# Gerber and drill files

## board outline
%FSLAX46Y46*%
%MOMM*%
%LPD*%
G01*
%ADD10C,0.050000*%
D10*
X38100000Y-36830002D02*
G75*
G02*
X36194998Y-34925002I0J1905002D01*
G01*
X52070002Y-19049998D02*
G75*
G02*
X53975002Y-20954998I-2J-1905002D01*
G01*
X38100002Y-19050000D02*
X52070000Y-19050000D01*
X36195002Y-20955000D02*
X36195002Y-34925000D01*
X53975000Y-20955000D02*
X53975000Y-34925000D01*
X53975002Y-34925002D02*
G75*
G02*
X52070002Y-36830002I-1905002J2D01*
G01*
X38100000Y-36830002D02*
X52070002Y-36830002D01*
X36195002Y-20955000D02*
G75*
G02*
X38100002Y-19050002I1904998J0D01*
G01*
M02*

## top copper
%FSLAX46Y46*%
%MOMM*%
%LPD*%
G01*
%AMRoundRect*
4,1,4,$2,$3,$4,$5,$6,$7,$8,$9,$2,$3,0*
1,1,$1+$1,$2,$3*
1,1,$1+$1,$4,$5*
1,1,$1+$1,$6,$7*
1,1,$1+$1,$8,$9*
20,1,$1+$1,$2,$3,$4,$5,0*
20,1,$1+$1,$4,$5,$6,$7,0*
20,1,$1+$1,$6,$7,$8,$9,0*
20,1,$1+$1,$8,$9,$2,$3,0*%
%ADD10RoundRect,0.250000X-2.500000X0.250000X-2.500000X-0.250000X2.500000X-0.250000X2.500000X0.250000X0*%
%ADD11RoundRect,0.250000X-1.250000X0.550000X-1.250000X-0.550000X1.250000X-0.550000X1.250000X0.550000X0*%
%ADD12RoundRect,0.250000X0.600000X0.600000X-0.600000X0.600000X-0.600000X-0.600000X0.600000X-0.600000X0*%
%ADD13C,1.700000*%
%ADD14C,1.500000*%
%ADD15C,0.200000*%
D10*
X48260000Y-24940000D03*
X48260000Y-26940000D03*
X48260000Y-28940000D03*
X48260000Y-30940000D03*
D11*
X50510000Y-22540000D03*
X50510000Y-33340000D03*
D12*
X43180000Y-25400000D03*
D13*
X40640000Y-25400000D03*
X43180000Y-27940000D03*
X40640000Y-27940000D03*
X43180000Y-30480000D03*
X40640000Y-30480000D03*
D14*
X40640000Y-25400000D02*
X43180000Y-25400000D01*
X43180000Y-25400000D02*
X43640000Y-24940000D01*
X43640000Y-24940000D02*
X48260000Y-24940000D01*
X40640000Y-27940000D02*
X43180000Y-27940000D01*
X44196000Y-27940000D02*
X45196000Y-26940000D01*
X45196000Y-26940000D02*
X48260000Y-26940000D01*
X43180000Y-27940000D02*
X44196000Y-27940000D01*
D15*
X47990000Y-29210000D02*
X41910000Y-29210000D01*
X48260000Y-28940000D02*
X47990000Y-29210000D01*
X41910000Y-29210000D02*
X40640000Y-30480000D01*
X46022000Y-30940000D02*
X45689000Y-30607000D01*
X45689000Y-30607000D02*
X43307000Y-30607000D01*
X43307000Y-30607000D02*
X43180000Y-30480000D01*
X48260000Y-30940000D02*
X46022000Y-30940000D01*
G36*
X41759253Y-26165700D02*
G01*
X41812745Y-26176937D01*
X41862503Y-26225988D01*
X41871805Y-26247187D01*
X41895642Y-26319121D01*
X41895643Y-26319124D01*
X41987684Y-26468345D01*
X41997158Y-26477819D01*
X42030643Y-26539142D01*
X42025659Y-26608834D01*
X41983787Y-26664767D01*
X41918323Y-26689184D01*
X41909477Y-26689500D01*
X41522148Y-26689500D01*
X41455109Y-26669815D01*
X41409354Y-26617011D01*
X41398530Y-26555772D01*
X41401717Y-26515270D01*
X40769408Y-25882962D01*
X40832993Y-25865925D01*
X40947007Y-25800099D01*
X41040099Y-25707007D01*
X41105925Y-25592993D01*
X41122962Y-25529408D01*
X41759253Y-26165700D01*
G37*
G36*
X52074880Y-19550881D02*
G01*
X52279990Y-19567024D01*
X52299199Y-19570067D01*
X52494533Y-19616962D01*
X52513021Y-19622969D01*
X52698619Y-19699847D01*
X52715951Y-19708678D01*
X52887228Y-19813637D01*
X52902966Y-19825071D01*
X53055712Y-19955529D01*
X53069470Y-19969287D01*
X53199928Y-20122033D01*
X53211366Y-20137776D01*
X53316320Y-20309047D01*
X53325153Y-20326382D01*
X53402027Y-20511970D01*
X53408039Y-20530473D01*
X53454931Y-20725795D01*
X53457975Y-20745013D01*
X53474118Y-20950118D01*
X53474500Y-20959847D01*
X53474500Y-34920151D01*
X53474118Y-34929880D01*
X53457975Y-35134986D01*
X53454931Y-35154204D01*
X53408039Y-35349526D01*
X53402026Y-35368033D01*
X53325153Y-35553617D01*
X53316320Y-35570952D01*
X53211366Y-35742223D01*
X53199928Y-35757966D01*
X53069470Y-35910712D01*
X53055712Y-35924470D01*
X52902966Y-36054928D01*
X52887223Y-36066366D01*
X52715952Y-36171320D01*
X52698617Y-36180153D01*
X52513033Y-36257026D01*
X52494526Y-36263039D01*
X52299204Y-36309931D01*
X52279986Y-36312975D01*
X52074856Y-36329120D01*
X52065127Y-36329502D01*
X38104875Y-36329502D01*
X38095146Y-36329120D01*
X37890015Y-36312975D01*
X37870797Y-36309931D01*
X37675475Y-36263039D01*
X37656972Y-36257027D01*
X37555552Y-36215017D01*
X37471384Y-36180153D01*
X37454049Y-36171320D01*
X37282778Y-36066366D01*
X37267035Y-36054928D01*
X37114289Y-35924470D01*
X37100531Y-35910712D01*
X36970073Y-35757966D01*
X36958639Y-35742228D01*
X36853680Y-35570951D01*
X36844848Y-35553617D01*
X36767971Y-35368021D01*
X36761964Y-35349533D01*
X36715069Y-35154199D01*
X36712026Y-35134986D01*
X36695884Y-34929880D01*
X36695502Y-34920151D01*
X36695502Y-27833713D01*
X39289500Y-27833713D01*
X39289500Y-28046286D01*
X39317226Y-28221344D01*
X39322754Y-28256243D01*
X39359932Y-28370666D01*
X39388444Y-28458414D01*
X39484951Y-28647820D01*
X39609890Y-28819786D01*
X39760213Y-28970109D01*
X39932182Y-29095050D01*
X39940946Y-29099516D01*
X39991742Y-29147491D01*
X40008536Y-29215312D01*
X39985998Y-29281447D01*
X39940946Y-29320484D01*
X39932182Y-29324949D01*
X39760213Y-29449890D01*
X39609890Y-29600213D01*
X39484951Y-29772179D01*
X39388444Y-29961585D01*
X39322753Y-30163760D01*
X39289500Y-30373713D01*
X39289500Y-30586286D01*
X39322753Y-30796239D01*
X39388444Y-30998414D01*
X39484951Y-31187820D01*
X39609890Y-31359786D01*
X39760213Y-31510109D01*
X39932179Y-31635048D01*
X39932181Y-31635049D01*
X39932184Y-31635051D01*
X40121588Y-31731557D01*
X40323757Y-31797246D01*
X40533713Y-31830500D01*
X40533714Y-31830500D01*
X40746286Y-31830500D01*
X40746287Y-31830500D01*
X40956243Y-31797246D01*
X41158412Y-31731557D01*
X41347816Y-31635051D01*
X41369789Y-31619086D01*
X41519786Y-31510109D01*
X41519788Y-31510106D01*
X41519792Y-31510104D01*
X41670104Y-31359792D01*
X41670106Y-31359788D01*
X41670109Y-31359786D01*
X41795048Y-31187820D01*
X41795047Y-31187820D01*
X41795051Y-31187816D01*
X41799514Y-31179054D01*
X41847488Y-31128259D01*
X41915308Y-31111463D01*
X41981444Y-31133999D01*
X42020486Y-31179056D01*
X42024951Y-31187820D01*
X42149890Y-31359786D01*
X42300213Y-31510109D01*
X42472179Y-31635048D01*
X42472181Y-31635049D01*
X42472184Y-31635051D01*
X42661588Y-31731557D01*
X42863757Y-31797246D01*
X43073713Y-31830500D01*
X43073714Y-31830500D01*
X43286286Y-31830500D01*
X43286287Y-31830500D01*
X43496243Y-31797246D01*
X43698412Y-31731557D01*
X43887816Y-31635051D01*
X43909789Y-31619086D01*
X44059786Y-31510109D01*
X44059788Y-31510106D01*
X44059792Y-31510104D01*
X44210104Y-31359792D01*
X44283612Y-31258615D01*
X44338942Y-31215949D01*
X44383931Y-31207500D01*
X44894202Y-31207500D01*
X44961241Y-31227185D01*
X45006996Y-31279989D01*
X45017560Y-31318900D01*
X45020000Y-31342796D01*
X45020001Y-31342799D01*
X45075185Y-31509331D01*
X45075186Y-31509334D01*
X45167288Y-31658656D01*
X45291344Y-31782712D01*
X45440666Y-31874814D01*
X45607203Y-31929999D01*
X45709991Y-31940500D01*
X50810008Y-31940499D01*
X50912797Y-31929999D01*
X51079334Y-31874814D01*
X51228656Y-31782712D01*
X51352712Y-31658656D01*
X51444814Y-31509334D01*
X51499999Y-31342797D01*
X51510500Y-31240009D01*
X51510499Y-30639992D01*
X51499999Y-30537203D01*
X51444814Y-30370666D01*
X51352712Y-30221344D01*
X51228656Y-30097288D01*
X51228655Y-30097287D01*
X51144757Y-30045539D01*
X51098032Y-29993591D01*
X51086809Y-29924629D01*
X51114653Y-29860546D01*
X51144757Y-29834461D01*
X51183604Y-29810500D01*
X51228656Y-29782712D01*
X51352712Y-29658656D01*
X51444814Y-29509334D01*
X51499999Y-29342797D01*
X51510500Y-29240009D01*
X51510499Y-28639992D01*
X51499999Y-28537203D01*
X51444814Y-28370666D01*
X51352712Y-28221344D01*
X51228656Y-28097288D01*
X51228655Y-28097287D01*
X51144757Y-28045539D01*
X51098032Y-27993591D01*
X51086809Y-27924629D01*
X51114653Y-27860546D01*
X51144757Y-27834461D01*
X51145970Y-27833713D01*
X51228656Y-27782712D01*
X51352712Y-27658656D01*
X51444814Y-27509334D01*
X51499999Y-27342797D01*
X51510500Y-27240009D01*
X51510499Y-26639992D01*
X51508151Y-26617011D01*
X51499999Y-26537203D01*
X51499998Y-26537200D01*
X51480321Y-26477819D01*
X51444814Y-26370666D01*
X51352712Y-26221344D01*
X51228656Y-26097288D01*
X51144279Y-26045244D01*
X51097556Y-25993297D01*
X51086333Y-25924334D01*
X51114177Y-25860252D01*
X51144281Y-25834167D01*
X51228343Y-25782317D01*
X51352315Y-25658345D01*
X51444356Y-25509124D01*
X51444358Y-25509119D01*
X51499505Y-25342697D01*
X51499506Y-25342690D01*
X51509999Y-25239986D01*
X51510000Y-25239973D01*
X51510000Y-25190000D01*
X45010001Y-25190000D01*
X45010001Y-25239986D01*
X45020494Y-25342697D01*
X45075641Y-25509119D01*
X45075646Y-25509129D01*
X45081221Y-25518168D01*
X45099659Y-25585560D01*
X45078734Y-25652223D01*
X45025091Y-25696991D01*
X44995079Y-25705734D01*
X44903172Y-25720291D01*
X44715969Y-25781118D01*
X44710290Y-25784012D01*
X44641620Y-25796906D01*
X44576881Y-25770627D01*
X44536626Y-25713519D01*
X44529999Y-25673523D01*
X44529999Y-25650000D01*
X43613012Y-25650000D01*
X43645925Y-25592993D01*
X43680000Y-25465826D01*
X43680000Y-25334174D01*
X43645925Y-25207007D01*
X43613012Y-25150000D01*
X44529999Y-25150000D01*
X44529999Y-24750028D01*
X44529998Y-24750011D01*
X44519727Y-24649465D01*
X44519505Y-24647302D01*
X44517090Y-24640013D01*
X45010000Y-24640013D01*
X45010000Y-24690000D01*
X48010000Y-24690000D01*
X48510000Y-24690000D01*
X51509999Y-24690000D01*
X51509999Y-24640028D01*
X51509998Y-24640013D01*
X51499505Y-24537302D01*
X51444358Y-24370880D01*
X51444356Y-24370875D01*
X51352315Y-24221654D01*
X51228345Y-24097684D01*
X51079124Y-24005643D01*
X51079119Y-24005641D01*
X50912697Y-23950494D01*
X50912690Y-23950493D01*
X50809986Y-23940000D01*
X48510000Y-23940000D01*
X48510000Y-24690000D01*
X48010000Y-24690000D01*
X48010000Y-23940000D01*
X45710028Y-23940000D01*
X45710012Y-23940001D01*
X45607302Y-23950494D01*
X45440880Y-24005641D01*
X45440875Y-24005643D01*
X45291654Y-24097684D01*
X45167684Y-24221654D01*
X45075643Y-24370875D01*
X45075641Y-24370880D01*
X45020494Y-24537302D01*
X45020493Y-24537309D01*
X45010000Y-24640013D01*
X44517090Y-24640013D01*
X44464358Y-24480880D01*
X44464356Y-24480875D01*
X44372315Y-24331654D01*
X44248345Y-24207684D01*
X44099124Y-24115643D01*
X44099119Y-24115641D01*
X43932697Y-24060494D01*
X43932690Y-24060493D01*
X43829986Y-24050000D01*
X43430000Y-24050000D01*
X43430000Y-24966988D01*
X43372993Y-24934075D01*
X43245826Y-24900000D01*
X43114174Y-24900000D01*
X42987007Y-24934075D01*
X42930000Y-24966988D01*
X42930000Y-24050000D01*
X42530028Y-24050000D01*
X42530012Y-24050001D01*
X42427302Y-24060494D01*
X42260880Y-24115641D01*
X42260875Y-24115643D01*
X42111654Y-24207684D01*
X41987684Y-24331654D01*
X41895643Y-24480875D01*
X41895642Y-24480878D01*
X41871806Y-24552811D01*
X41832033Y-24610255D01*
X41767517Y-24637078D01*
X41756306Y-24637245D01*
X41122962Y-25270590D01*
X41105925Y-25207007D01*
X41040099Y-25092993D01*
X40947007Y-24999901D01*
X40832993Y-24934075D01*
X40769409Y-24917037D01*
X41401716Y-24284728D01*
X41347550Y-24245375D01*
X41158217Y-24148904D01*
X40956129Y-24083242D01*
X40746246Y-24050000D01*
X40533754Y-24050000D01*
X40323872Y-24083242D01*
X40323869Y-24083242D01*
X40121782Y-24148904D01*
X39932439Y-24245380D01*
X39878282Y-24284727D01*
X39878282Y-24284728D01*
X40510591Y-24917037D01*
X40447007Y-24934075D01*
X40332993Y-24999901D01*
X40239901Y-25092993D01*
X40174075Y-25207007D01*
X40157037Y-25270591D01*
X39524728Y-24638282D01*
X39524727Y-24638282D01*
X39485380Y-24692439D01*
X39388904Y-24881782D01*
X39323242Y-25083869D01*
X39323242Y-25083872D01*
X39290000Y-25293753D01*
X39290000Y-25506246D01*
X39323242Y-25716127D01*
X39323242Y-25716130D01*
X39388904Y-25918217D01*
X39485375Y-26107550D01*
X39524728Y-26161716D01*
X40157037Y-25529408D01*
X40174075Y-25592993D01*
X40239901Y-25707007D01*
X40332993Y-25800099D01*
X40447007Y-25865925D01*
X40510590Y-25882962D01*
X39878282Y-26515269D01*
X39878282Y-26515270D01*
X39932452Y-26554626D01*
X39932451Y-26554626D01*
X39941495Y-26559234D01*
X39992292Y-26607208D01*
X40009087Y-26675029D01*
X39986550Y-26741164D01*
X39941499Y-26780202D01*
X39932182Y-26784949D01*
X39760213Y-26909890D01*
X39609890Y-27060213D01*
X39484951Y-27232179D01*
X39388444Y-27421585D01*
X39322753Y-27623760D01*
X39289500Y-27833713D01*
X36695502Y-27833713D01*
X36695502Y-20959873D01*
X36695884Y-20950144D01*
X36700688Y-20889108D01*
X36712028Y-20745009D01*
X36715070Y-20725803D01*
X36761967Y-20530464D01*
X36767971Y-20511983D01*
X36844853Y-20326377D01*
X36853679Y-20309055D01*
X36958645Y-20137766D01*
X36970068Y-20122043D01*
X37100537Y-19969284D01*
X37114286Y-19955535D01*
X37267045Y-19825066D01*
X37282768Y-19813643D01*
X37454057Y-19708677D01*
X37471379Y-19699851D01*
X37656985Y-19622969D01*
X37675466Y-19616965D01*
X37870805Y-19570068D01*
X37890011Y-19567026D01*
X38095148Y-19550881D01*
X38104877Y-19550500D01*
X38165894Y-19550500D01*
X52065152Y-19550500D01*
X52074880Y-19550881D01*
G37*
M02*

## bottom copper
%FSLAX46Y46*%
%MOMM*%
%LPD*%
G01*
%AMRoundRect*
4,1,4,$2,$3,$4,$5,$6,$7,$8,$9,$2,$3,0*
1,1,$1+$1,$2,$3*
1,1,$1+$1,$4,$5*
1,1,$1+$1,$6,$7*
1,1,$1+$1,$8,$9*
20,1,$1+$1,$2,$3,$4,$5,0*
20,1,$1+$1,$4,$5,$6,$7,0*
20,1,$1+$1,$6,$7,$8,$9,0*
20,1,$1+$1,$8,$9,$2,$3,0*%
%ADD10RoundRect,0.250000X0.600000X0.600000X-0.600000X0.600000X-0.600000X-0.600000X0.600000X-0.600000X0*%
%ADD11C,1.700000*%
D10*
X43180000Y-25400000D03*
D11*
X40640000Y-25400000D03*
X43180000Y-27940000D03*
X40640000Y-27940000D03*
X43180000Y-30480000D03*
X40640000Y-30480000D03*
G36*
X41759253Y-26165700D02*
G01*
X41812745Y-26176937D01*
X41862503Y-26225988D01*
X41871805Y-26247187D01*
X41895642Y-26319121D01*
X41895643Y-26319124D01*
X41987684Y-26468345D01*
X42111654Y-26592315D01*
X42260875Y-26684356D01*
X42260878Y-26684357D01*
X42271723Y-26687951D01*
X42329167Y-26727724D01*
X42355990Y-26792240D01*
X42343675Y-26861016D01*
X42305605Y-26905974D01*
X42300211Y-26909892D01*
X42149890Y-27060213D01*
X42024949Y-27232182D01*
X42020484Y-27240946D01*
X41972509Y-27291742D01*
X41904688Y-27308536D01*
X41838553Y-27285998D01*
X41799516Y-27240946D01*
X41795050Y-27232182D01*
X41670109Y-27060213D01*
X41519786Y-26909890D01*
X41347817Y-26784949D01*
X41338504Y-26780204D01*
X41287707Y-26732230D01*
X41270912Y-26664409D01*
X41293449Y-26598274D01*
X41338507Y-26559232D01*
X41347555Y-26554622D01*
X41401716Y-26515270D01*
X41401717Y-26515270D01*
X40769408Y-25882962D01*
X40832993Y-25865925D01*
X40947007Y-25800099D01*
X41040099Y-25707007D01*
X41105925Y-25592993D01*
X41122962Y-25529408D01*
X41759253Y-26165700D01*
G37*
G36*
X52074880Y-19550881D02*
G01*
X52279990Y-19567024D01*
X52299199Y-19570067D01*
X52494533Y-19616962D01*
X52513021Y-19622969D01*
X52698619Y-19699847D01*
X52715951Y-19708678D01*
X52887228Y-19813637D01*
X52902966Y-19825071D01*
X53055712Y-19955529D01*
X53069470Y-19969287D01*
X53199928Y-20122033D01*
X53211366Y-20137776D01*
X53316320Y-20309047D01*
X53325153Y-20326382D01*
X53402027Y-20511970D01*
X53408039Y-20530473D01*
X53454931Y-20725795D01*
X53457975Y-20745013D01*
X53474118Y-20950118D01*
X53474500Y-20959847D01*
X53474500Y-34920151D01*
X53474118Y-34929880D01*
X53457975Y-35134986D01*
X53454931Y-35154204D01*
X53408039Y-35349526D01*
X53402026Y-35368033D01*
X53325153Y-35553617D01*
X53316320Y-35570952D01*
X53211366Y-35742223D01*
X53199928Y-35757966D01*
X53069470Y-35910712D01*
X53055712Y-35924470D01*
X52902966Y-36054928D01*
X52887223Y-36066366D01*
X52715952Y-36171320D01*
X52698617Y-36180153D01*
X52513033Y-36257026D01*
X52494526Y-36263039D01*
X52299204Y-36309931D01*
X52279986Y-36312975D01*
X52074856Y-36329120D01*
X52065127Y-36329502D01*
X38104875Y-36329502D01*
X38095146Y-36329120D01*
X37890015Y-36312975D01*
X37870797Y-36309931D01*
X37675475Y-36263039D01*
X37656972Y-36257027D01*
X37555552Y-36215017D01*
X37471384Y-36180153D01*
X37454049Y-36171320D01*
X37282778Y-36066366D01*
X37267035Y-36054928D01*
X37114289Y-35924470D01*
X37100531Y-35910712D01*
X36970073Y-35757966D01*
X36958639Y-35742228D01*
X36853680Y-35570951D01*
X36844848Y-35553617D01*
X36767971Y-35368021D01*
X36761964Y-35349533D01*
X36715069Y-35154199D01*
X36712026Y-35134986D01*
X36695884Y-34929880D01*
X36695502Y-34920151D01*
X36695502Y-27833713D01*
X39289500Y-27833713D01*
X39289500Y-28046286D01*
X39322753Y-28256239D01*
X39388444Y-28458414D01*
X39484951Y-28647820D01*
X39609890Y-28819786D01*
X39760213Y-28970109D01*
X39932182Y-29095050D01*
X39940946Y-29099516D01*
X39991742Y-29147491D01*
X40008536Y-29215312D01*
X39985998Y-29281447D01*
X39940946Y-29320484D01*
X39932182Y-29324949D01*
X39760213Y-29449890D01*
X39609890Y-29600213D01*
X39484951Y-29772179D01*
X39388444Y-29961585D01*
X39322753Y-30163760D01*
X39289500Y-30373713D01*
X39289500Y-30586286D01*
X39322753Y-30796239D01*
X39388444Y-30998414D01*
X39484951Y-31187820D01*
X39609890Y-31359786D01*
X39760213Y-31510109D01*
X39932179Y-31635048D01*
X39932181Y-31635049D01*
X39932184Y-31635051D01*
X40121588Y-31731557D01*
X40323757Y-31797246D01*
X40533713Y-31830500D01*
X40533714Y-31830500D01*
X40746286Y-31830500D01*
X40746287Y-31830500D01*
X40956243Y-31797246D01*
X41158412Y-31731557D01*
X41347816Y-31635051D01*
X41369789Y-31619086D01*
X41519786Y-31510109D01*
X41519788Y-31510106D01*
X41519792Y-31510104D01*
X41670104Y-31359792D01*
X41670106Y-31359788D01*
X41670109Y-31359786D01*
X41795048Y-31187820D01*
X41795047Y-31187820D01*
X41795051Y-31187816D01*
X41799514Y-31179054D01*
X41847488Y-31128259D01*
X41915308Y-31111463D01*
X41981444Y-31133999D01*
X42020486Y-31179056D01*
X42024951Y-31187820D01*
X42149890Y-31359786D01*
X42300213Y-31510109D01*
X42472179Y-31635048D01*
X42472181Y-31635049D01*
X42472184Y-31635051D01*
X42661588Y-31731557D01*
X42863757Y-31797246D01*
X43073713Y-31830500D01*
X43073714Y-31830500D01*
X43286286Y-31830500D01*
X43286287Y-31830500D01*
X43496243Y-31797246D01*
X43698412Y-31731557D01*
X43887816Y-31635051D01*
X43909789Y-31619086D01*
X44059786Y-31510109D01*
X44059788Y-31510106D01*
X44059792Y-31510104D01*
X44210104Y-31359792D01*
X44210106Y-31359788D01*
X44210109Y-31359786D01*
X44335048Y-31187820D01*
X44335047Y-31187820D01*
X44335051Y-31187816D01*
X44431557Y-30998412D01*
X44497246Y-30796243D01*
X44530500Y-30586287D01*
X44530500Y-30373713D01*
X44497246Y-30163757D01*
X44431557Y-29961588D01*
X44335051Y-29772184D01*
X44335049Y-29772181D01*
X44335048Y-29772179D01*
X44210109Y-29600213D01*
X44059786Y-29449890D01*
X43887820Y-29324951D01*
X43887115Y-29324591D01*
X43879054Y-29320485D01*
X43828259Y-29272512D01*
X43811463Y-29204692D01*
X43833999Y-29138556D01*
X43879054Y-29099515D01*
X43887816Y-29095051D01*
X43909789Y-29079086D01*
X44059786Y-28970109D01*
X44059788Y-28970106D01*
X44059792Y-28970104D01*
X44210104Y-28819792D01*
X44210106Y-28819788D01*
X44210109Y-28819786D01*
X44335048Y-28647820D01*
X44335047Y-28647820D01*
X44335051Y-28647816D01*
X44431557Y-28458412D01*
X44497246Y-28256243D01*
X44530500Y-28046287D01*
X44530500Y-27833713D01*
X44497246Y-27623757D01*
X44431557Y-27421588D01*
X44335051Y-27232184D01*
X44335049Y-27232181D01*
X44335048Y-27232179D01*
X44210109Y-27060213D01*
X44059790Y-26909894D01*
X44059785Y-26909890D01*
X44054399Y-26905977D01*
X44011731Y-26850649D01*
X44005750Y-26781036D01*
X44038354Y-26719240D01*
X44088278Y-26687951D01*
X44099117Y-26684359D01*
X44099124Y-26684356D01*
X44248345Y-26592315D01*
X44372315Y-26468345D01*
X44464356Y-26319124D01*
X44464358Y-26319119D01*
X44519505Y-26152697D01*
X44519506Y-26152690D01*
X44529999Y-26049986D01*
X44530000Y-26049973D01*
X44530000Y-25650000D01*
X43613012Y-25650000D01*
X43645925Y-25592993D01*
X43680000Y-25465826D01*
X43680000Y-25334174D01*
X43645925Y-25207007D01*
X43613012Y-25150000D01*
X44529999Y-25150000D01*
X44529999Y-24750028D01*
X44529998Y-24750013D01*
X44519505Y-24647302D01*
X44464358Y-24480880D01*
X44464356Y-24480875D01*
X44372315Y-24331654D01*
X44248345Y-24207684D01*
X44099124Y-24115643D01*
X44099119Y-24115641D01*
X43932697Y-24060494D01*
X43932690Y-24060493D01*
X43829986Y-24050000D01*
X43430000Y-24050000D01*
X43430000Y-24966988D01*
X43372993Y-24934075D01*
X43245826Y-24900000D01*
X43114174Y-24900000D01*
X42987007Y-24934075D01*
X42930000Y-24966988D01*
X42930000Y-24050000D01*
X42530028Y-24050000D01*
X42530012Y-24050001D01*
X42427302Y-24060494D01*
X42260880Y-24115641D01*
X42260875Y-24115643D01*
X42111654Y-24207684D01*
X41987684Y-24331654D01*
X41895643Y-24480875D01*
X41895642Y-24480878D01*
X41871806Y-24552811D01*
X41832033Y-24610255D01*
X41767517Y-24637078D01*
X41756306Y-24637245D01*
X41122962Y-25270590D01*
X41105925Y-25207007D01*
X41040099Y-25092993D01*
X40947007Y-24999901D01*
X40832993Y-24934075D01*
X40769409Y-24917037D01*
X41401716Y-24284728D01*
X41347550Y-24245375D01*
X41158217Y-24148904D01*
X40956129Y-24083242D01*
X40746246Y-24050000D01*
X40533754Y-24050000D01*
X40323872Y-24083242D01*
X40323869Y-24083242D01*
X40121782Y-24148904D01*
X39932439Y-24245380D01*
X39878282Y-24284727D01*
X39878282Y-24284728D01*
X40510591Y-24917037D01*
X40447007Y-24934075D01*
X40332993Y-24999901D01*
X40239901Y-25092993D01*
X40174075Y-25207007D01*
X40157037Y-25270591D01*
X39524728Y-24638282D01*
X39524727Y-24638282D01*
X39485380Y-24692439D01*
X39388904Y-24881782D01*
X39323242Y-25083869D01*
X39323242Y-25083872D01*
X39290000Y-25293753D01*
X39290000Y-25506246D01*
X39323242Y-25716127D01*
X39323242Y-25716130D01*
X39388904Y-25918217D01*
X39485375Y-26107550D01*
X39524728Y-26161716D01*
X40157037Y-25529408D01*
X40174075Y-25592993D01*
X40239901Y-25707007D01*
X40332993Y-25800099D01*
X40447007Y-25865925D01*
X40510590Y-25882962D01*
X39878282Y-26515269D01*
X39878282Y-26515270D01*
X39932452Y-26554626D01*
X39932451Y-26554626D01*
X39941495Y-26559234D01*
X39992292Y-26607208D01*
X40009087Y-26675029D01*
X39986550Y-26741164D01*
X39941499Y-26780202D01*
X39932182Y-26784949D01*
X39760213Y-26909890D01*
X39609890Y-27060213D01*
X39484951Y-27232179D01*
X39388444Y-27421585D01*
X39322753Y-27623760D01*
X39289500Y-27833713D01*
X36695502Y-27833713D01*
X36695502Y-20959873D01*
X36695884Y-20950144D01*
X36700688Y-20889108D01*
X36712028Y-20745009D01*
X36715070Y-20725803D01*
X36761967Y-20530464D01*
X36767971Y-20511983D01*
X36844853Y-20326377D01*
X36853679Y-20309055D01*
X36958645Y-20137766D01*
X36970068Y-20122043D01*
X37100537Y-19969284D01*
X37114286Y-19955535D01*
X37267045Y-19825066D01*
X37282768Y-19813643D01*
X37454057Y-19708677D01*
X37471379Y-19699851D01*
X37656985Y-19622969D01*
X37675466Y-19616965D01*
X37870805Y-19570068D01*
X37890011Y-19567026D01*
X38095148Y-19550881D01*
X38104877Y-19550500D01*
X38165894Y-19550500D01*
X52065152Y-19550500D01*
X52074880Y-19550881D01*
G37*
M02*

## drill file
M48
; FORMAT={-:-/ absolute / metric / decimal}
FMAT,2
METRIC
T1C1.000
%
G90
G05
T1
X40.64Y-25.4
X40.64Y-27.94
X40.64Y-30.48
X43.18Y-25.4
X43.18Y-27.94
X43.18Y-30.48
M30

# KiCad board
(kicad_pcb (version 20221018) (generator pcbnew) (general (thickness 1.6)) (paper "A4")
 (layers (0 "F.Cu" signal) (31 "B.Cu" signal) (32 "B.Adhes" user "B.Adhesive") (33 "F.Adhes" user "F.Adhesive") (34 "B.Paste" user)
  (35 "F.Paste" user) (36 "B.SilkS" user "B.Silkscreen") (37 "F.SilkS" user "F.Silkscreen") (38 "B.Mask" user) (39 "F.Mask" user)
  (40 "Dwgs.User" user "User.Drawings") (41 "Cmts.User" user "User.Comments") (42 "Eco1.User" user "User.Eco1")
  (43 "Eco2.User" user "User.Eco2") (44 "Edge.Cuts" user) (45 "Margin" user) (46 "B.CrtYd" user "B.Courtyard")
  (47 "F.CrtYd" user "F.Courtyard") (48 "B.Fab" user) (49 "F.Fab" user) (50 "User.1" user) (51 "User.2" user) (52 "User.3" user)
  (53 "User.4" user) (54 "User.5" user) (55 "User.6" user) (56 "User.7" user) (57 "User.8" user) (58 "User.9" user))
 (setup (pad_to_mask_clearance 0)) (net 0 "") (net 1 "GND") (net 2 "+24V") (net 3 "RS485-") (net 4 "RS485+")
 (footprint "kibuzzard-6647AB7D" (layer "F.Cu") (at 41.148 34.671)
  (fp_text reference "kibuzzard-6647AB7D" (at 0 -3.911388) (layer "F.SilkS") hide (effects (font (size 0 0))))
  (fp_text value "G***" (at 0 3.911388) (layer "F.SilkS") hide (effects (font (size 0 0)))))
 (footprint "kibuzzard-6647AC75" (layer "F.Cu") (at 52.324 27.94 90)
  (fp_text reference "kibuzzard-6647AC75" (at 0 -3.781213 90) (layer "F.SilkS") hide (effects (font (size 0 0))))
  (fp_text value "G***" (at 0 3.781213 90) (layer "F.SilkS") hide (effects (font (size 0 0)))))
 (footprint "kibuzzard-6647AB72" (layer "F.Cu") (at 41.783 21.082)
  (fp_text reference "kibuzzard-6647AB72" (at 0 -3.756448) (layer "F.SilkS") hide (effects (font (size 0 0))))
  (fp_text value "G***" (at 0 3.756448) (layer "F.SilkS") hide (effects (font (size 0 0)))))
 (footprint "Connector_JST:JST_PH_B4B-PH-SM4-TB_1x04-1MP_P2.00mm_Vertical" (layer "F.Cu") (at 48.76 27.94 -90)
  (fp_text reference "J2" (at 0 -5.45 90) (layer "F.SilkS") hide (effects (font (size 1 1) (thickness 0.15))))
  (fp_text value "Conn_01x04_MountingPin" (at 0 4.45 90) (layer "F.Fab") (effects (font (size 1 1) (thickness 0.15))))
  (pad "1" smd roundrect (at -3 0.5 270) (size 1 5.5) (layers "F.Cu" "F.Paste" "F.Mask") (roundrect_rratio 0.25) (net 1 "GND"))
  (pad "2" smd roundrect (at -1 0.5 270) (size 1 5.5) (layers "F.Cu" "F.Paste" "F.Mask") (roundrect_rratio 0.25) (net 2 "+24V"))
  (pad "3" smd roundrect (at 1 0.5 270) (size 1 5.5) (layers "F.Cu" "F.Paste" "F.Mask") (roundrect_rratio 0.25) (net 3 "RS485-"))
  (pad "4" smd roundrect (at 3 0.5 270) (size 1 5.5) (layers "F.Cu" "F.Paste" "F.Mask") (roundrect_rratio 0.25) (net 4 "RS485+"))
  (pad "MP" smd roundrect (at -5.4 -1.75 270) (size 1.6 3) (layers "F.Cu" "F.Paste" "F.Mask") (roundrect_rratio 0.15625) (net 1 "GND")
   (zone_connect 2))
  (pad "MP" smd roundrect (at 5.4 -1.75 270) (size 1.6 3) (layers "F.Cu" "F.Paste" "F.Mask") (roundrect_rratio 0.15625) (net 1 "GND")
   (zone_connect 2)))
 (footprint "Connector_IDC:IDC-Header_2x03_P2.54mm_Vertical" (layer "B.Cu") (at 43.18 25.4 180)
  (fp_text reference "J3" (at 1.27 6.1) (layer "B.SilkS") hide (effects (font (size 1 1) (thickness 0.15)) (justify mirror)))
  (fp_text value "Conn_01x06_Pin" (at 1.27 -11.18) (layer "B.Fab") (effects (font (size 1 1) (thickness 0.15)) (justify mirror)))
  (pad "1" thru_hole roundrect (at 0 0 180) (size 1.7 1.7) (drill 1) (layers "*.Cu" "*.Mask") (roundrect_rratio 0.1470588235) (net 1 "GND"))
  (pad "2" thru_hole circle (at 2.54 0 180) (size 1.7 1.7) (drill 1) (layers "*.Cu" "*.Mask") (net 1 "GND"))
  (pad "3" thru_hole circle (at 0 -2.54 180) (size 1.7 1.7) (drill 1) (layers "*.Cu" "*.Mask") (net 2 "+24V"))
  (pad "4" thru_hole circle (at 2.54 -2.54 180) (size 1.7 1.7) (drill 1) (layers "*.Cu" "*.Mask") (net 2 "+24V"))
  (pad "5" thru_hole circle (at 0 -5.08 180) (size 1.7 1.7) (drill 1) (layers "*.Cu" "*.Mask") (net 4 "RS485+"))
  (pad "6" thru_hole circle (at 2.54 -5.08 180) (size 1.7 1.7) (drill 1) (layers "*.Cu" "*.Mask") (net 3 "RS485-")))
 (gr_arc (start 38.1 36.830002) (mid 36.752962 36.27204) (end 36.195 34.925002) (stroke (width 0.05) (type default)) (layer "Edge.Cuts"))
 (gr_arc (start 52.070002 19.049998) (mid 53.41704 19.60796) (end 53.975002 20.954998) (stroke (width 0.05) (type default))
  (layer "Edge.Cuts"))
 (gr_line (start 38.100002 19.05) (end 52.07 19.05) (stroke (width 0.05) (type default)) (layer "Edge.Cuts"))
 (gr_line (start 36.195002 20.955) (end 36.195002 34.925) (stroke (width 0.05) (type default)) (layer "Edge.Cuts"))
 (gr_line (start 53.975 20.955) (end 53.975 34.925) (stroke (width 0.05) (type default)) (layer "Edge.Cuts"))
 (gr_arc (start 53.975002 34.925002) (mid 53.41704 36.27204) (end 52.070002 36.830002) (stroke (width 0.05) (type default))
  (layer "Edge.Cuts"))
 (gr_line (start 38.1 36.830002) (end 52.070002 36.830002) (stroke (width 0.05) (type default)) (layer "Edge.Cuts"))
 (gr_arc (start 36.195002 20.955) (mid 36.752964 19.607962) (end 38.100002 19.05) (stroke (width 0.05) (type default)) (layer "Edge.Cuts"))
 (segment (start 40.64 25.4) (end 43.18 25.4) (width 1.5) (layer "F.Cu") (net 1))
 (segment (start 43.18 25.4) (end 43.64 24.94) (width 1.5) (layer "F.Cu") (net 1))
 (segment (start 43.64 24.94) (end 48.26 24.94) (width 1.5) (layer "F.Cu") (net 1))
 (segment (start 40.64 27.94) (end 43.18 27.94) (width 1.5) (layer "F.Cu") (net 2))
 (segment (start 44.196 27.94) (end 45.196 26.94) (width 1.5) (layer "F.Cu") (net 2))
 (segment (start 45.196 26.94) (end 48.26 26.94) (width 1.5) (layer "F.Cu") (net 2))
 (segment (start 43.18 27.94) (end 44.196 27.94) (width 1.5) (layer "F.Cu") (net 2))
 (segment (start 47.99 29.21) (end 41.91 29.21) (width 0.2) (layer "F.Cu") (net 3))
 (segment (start 48.26 28.94) (end 47.99 29.21) (width 0.2) (layer "F.Cu") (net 3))
 (segment (start 41.91 29.21) (end 40.64 30.48) (width 0.2) (layer "F.Cu") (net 3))
 (segment (start 46.022 30.94) (end 45.689 30.607) (width 0.2) (layer "F.Cu") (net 4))
 (segment (start 45.689 30.607) (end 43.307 30.607) (width 0.2) (layer "F.Cu") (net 4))
 (segment (start 43.307 30.607) (end 43.18 30.48) (width 0.2) (layer "F.Cu") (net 4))
 (segment (start 48.26 30.94) (end 46.022 30.94) (width 0.2) (layer "F.Cu") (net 4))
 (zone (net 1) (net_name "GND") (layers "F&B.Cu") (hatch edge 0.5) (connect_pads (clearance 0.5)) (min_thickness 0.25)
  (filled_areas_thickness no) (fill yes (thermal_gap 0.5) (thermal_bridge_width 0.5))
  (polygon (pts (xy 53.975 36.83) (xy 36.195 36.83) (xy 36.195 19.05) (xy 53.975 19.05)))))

